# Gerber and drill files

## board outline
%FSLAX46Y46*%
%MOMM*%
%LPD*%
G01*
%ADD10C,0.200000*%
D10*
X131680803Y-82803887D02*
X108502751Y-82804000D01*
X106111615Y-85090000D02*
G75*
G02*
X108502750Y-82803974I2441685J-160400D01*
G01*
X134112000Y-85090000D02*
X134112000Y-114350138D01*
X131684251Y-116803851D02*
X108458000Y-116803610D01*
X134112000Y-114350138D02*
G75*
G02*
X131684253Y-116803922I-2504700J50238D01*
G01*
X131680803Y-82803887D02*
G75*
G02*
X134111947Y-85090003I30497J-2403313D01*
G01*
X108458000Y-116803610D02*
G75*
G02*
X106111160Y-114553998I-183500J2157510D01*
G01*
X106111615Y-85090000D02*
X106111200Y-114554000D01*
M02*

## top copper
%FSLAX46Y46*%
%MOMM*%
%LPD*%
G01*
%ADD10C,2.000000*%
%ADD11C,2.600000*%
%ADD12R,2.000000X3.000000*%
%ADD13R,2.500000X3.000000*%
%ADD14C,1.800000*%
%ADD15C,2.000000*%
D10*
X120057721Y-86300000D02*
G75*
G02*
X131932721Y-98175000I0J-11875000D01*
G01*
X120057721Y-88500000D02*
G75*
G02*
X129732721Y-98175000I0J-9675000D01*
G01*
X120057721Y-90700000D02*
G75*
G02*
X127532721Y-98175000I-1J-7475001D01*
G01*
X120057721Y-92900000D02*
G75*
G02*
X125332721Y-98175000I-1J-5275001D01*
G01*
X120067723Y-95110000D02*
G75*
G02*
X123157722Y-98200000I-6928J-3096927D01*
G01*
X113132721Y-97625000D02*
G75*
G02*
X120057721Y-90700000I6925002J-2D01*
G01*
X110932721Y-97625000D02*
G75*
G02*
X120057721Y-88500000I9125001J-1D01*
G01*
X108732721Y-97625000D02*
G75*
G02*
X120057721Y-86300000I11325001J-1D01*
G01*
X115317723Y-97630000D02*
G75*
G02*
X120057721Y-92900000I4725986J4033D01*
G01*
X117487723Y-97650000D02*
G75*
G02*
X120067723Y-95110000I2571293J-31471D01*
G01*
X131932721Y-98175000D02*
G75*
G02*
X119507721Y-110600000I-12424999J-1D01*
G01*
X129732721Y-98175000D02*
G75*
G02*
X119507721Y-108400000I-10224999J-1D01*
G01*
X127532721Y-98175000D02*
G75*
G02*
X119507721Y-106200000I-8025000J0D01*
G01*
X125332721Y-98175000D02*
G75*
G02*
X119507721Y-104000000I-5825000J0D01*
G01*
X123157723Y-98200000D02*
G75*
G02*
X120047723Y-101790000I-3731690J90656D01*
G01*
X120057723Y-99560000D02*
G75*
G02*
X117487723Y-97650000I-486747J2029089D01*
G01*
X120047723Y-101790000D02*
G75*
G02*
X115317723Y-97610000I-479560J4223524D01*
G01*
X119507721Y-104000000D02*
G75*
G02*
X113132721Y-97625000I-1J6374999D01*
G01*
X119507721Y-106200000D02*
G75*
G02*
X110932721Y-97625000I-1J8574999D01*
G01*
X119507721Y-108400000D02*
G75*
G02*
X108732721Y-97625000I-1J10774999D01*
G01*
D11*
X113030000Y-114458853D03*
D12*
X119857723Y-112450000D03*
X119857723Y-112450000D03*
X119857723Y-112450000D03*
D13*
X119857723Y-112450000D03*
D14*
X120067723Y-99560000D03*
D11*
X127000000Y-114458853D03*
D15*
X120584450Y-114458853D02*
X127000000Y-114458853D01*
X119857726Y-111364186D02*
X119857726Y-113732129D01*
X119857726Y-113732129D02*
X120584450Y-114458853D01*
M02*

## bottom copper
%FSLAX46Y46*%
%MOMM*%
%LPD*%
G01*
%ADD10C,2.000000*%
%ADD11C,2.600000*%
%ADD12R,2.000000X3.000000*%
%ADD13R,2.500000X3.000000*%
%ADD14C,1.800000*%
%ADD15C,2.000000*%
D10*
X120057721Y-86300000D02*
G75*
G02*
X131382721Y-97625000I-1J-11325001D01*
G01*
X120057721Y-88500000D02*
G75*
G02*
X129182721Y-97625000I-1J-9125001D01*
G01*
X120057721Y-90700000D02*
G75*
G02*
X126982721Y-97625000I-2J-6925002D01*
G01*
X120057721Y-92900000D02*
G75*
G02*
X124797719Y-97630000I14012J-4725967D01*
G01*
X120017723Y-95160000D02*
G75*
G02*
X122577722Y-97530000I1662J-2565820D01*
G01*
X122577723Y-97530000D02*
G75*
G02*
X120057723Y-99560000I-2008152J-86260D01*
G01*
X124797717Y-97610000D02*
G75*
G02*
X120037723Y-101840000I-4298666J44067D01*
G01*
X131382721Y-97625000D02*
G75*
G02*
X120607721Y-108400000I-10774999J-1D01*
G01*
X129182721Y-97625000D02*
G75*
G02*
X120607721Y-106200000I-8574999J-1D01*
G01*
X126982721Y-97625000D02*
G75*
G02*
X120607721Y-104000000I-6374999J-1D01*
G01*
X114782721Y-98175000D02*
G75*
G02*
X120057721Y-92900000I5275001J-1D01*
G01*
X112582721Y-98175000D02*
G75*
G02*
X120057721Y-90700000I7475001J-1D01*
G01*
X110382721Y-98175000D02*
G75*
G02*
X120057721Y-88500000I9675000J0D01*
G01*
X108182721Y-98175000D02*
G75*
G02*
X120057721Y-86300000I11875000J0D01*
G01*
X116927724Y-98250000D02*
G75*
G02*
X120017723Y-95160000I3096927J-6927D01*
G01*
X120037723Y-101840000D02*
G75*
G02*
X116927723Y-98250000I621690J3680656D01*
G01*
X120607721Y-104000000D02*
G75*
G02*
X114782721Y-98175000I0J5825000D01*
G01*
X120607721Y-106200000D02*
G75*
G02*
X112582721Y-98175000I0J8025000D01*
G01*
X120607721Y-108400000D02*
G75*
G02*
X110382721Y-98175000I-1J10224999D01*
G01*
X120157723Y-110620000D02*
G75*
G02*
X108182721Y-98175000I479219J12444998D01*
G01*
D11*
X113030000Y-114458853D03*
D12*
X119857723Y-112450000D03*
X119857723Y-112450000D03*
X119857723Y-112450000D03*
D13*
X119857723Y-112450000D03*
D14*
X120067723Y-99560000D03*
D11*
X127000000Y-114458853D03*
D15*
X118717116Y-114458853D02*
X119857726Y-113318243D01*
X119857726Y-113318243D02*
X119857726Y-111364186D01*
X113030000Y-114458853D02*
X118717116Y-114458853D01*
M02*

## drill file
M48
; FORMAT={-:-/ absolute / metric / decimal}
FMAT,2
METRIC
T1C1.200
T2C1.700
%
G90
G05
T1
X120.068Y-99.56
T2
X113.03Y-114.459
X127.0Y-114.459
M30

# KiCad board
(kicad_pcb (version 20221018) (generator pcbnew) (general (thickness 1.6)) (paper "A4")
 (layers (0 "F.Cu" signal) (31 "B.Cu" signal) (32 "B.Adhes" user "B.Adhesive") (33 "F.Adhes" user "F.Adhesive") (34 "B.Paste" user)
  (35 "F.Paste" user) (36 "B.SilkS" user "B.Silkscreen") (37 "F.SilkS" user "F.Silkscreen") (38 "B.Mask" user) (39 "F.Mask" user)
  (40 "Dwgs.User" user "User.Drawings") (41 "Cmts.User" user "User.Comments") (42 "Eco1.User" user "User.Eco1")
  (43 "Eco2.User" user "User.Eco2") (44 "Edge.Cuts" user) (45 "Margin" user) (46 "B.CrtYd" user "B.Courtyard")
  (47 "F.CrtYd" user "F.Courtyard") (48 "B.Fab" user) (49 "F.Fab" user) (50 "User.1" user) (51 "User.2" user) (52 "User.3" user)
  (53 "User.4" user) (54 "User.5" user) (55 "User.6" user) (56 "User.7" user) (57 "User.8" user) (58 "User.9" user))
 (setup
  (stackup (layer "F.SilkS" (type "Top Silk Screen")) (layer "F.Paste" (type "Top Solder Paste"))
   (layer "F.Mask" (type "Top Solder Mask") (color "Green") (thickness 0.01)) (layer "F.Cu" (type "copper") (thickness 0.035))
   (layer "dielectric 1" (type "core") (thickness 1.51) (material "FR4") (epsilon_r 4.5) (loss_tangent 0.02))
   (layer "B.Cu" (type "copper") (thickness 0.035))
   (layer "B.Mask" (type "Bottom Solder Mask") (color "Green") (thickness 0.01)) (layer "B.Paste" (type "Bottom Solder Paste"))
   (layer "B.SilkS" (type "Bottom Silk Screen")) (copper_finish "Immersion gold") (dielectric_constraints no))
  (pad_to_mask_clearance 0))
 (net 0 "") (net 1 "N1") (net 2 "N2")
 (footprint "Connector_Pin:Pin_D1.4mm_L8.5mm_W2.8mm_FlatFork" (layer "F.Cu") (at 113.03 114.458853)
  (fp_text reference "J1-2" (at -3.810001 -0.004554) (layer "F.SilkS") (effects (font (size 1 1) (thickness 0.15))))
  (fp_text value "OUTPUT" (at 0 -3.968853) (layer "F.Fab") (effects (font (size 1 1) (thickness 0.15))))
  (pad "1" thru_hole circle (at 0 0) (size 2.6 2.6) (drill 1.7) (layers "*.Cu" "*.Mask") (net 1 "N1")))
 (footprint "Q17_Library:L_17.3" (layer "F.Cu") (at 120.057723 98.2 -90) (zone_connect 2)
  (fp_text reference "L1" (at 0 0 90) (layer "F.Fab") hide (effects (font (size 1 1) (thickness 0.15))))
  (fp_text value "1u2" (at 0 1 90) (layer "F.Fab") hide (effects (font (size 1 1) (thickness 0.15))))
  (fp_arc (start -11.9 0.000002) (mid -8.421893 -8.396891) (end -0.025 -11.874998) (stroke (width 2) (type solid)) (layer "F.Cu"))
  (fp_arc (start -9.7 0.000002) (mid -6.866258 -6.841256) (end -0.025 -9.674998) (stroke (width 2) (type solid)) (layer "F.Cu"))
  (fp_arc (start -7.5 0.000002) (mid -5.310623 -5.285621) (end -0.025 -7.474998) (stroke (width 2) (type solid)) (layer "F.Cu"))
  (fp_arc (start -5.3 0.000002) (mid -3.754988 -3.729986) (end -0.025 -5.274998) (stroke (width 2) (type solid)) (layer "F.Cu"))
  (fp_arc (start -3.09 -0.01) (mid -2.182936 -2.192936) (end 0 -3.099999) (stroke (width 2) (type solid)) (layer "F.Cu"))
  (fp_arc (start -0.575 6.925002) (mid -5.471714 4.896716) (end -7.5 0.000002) (stroke (width 2) (type solid)) (layer "F.Cu"))
  (fp_arc (start -0.575 9.125002) (mid -7.027349 6.452351) (end -9.7 0.000002) (stroke (width 2) (type solid)) (layer "F.Cu"))
  (fp_arc (start -0.575 11.325002) (mid -8.582984 8.007986) (end -11.9 0.000002) (stroke (width 2) (type solid)) (layer "F.Cu"))
  (fp_arc (start -0.57 4.74) (mid -3.919337 3.352262) (end -5.3 0.000002) (stroke (width 2) (type solid)) (layer "F.Cu"))
  (fp_arc (start -0.55 2.57) (mid -2.350994 1.802761) (end -3.09 -0.01) (stroke (width 2) (type solid)) (layer "F.Cu"))
  (fp_arc (start -0.025 -11.874998) (mid 8.760802 -8.2358) (end 12.4 0.550002) (stroke (width 2) (type solid)) (layer "F.Cu"))
  (fp_arc (start -0.025 -9.674998) (mid 7.205167 -6.680165) (end 10.2 0.550002) (stroke (width 2) (type solid)) (layer "F.Cu"))
  (fp_arc (start -0.025 -7.474998) (mid 5.649532 -5.12453) (end 8 0.550002) (stroke (width 2) (type solid)) (layer "F.Cu"))
  (fp_arc (start -0.025 -5.274998) (mid 4.093897 -3.568895) (end 5.8 0.550002) (stroke (width 2) (type solid)) (layer "F.Cu"))
  (fp_arc (start 0 -3.1) (mid 2.353464 -2.189658) (end 3.59 0.01) (stroke (width 2) (type solid)) (layer "F.Cu"))
  (fp_arc (start 1.36 0) (mid 1.005692 1.731429) (end -0.55 2.57) (stroke (width 2) (type solid)) (layer "F.Cu"))
  (fp_arc (start 3.59 0.01) (mid 2.551621 3.304339) (end -0.59 4.739999) (stroke (width 2) (type solid)) (layer "F.Cu"))
  (fp_arc (start 5.8 0.550002) (mid 3.932806 5.057808) (end -0.575 6.925002) (stroke (width 2) (type solid)) (layer "F.Cu"))
  (fp_arc (start 8 0.550002) (mid 5.488441 6.613443) (end -0.575 9.125002) (stroke (width 2) (type solid)) (layer "F.Cu"))
  (fp_arc (start 10.2 0.550002) (mid 7.044076 8.169078) (end -0.575 11.325002) (stroke (width 2) (type solid)) (layer "F.Cu"))
  (fp_arc (start -11.9 0.000002) (mid -8.582984 -8.007982) (end -0.575 -11.324998) (stroke (width 2) (type solid)) (layer "B.Cu"))
  (fp_arc (start -9.7 0.000002) (mid -7.027349 -6.452347) (end -0.575 -9.124998) (stroke (width 2) (type solid)) (layer "B.Cu"))
  (fp_arc (start -7.5 0.000002) (mid -5.471714 -4.896712) (end -0.575 -6.924998) (stroke (width 2) (type solid)) (layer "B.Cu"))
  (fp_arc (start -5.3 0.000002) (mid -3.919337 -3.352258) (end -0.57 -4.739996) (stroke (width 2) (type solid)) (layer "B.Cu"))
  (fp_arc (start -3.04 0.04) (mid -2.357014 -1.704755) (end -0.67 -2.52) (stroke (width 2) (type solid)) (layer "B.Cu"))
  (fp_arc (start -0.67 -2.52) (mid 0.981558 -1.772783) (end 1.36 0) (stroke (width 2) (type solid)) (layer "B.Cu"))
  (fp_arc (start -0.59 -4.739994) (mid 2.579336 -3.296939) (end 3.64 0.02) (stroke (width 2) (type solid)) (layer "B.Cu"))
  (fp_arc (start -0.575 -11.324998) (mid 7.044076 -8.169074) (end 10.2 -0.549998) (stroke (width 2) (type solid)) (layer "B.Cu"))
  (fp_arc (start -0.575 -9.124998) (mid 5.488441 -6.613439) (end 8 -0.549998) (stroke (width 2) (type solid)) (layer "B.Cu"))
  (fp_arc (start -0.575 -6.924998) (mid 3.932806 -5.057804) (end 5.8 -0.549998) (stroke (width 2) (type solid)) (layer "B.Cu"))
  (fp_arc (start -0.025 5.275002) (mid -3.754988 3.72999) (end -5.3 0.000002) (stroke (width 2) (type solid)) (layer "B.Cu"))
  (fp_arc (start -0.025 7.475002) (mid -5.310623 5.285625) (end -7.5 0.000002) (stroke (width 2) (type solid)) (layer "B.Cu"))
  (fp_arc (start -0.025 9.675002) (mid -6.866258 6.84126) (end -9.7 0.000002) (stroke (width 2) (type solid)) (layer "B.Cu"))
  (fp_arc (start -0.025 11.875002) (mid -8.421893 8.396895) (end -11.9 0.000002) (stroke (width 2) (type solid)) (layer "B.Cu"))
  (fp_arc (start 0.05 3.129999) (mid -2.132936 2.222936) (end -3.04 0.04) (stroke (width 2) (type solid)) (layer "B.Cu"))
  (fp_arc (start 3.64 0.02) (mid 2.403464 2.219658) (end 0.05 3.13) (stroke (width 2) (type solid)) (layer "B.Cu"))
  (fp_arc (start 5.8 -0.549998) (mid 4.093897 3.568899) (end -0.025 5.275002) (stroke (width 2) (type solid)) (layer "B.Cu"))
  (fp_arc (start 8 -0.549998) (mid 5.649532 5.124534) (end -0.025 7.475002) (stroke (width 2) (type solid)) (layer "B.Cu"))
  (fp_arc (start 10.2 -0.549998) (mid 7.205167 6.680169) (end -0.025 9.675002) (stroke (width 2) (type solid)) (layer "B.Cu"))
  (fp_arc (start 12.42 -0.1) (mid 8.610374 8.395076) (end -0.025 11.875002) (stroke (width 2) (type solid)) (layer "B.Cu"))
  (pad "1" smd rect (at 14.25 0.2 90) (size 3 2) (layers "*.Mask" "F.Cu" "F.Paste") (zone_connect 2))
  (pad "1" smd rect (at 14.25 0.2 90) (size 3 2) (layers "*.Mask" "F.Cu" "F.Paste") (zone_connect 2))
  (pad "1" smd rect (at 14.25 0.2 90) (size 3 2) (layers "*.Mask" "F.Cu" "F.Paste") (zone_connect 2))
  (pad "1" smd rect (at 14.25 0.2 90) (size 3 2.5) (layers "*.Mask" "F.Cu" "F.Paste") (zone_connect 2))
  (pad "2" smd rect (at 14.25 0.2 90) (size 3 2) (layers "B.Cu" "B.Paste" "B.Mask") (zone_connect 2))
  (pad "2" smd rect (at 14.25 0.2 90) (size 3 2) (layers "B.Cu" "B.Paste" "B.Mask") (zone_connect 2))
  (pad "2" smd rect (at 14.25 0.2 90) (size 3 2) (layers "B.Cu" "B.Paste" "B.Mask") (zone_connect 2))
  (pad "2" smd rect (at 14.25 0.2 90) (size 3 2.5) (layers "B.Cu" "B.Paste" "B.Mask") (zone_connect 2))
  (pad "lc" thru_hole circle (at 1.36 -0.01 90) (size 1.8 1.8) (drill 1.2) (layers "*.Cu" "*.Mask") (zone_connect 2)))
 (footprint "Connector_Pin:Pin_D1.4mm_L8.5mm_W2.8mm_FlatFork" (layer "F.Cu") (at 127 114.458853)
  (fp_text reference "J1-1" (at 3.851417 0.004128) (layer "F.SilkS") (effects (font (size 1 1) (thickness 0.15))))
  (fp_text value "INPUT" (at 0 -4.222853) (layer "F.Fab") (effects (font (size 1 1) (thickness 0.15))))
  (pad "1" thru_hole circle (at 0 0) (size 2.6 2.6) (drill 1.7) (layers "*.Cu" "*.Mask") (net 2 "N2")))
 (gr_line (start 131.680803 82.803887) (end 108.502751 82.804) (stroke (width 0.2) (type solid)) (layer "Edge.Cuts"))
 (gr_arc (start 106.111615 85.09) (mid 106.86236 83.481719) (end 108.502751 82.804) (stroke (width 0.2) (type solid)) (layer "Edge.Cuts"))
 (gr_line (start 134.112 85.09) (end 134.112 114.350138) (stroke (width 0.2) (type solid)) (layer "Edge.Cuts"))
 (gr_line (start 131.684251 116.803851) (end 108.458 116.80361) (stroke (width 0.2) (type solid)) (layer "Edge.Cuts"))
 (gr_arc (start 134.112 114.350138) (mid 133.388153 116.061837) (end 131.684251 116.803851) (stroke (width 0.2) (type solid))
  (layer "Edge.Cuts"))
 (gr_arc (start 131.680803 82.803887) (mid 133.357835 83.456226) (end 134.112 85.09) (stroke (width 0.2) (type solid)) (layer "Edge.Cuts"))
 (gr_arc (start 108.458 116.80361) (mid 106.77615 116.209221) (end 106.1112 114.554) (stroke (width 0.2) (type solid)) (layer "Edge.Cuts"))
 (gr_line (start 106.111615 85.09) (end 106.1112 114.554) (stroke (width 0.2) (type solid)) (layer "Edge.Cuts"))
 (segment (start 120.58445 114.458853) (end 127 114.458853) (width 2) (layer "F.Cu") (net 2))
 (segment (start 119.857726 111.364186) (end 119.857726 113.732129) (width 2) (layer "F.Cu") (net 2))
 (segment (start 119.857726 113.732129) (end 120.58445 114.458853) (width 2) (layer "F.Cu") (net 2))
 (segment (start 118.717116 114.458853) (end 119.857726 113.318243) (width 2) (layer "B.Cu") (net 1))
 (segment (start 119.857726 113.318243) (end 119.857726 111.364186) (width 2) (layer "B.Cu") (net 1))
 (segment (start 113.03 114.458853) (end 118.717116 114.458853) (width 2) (layer "B.Cu") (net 1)))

